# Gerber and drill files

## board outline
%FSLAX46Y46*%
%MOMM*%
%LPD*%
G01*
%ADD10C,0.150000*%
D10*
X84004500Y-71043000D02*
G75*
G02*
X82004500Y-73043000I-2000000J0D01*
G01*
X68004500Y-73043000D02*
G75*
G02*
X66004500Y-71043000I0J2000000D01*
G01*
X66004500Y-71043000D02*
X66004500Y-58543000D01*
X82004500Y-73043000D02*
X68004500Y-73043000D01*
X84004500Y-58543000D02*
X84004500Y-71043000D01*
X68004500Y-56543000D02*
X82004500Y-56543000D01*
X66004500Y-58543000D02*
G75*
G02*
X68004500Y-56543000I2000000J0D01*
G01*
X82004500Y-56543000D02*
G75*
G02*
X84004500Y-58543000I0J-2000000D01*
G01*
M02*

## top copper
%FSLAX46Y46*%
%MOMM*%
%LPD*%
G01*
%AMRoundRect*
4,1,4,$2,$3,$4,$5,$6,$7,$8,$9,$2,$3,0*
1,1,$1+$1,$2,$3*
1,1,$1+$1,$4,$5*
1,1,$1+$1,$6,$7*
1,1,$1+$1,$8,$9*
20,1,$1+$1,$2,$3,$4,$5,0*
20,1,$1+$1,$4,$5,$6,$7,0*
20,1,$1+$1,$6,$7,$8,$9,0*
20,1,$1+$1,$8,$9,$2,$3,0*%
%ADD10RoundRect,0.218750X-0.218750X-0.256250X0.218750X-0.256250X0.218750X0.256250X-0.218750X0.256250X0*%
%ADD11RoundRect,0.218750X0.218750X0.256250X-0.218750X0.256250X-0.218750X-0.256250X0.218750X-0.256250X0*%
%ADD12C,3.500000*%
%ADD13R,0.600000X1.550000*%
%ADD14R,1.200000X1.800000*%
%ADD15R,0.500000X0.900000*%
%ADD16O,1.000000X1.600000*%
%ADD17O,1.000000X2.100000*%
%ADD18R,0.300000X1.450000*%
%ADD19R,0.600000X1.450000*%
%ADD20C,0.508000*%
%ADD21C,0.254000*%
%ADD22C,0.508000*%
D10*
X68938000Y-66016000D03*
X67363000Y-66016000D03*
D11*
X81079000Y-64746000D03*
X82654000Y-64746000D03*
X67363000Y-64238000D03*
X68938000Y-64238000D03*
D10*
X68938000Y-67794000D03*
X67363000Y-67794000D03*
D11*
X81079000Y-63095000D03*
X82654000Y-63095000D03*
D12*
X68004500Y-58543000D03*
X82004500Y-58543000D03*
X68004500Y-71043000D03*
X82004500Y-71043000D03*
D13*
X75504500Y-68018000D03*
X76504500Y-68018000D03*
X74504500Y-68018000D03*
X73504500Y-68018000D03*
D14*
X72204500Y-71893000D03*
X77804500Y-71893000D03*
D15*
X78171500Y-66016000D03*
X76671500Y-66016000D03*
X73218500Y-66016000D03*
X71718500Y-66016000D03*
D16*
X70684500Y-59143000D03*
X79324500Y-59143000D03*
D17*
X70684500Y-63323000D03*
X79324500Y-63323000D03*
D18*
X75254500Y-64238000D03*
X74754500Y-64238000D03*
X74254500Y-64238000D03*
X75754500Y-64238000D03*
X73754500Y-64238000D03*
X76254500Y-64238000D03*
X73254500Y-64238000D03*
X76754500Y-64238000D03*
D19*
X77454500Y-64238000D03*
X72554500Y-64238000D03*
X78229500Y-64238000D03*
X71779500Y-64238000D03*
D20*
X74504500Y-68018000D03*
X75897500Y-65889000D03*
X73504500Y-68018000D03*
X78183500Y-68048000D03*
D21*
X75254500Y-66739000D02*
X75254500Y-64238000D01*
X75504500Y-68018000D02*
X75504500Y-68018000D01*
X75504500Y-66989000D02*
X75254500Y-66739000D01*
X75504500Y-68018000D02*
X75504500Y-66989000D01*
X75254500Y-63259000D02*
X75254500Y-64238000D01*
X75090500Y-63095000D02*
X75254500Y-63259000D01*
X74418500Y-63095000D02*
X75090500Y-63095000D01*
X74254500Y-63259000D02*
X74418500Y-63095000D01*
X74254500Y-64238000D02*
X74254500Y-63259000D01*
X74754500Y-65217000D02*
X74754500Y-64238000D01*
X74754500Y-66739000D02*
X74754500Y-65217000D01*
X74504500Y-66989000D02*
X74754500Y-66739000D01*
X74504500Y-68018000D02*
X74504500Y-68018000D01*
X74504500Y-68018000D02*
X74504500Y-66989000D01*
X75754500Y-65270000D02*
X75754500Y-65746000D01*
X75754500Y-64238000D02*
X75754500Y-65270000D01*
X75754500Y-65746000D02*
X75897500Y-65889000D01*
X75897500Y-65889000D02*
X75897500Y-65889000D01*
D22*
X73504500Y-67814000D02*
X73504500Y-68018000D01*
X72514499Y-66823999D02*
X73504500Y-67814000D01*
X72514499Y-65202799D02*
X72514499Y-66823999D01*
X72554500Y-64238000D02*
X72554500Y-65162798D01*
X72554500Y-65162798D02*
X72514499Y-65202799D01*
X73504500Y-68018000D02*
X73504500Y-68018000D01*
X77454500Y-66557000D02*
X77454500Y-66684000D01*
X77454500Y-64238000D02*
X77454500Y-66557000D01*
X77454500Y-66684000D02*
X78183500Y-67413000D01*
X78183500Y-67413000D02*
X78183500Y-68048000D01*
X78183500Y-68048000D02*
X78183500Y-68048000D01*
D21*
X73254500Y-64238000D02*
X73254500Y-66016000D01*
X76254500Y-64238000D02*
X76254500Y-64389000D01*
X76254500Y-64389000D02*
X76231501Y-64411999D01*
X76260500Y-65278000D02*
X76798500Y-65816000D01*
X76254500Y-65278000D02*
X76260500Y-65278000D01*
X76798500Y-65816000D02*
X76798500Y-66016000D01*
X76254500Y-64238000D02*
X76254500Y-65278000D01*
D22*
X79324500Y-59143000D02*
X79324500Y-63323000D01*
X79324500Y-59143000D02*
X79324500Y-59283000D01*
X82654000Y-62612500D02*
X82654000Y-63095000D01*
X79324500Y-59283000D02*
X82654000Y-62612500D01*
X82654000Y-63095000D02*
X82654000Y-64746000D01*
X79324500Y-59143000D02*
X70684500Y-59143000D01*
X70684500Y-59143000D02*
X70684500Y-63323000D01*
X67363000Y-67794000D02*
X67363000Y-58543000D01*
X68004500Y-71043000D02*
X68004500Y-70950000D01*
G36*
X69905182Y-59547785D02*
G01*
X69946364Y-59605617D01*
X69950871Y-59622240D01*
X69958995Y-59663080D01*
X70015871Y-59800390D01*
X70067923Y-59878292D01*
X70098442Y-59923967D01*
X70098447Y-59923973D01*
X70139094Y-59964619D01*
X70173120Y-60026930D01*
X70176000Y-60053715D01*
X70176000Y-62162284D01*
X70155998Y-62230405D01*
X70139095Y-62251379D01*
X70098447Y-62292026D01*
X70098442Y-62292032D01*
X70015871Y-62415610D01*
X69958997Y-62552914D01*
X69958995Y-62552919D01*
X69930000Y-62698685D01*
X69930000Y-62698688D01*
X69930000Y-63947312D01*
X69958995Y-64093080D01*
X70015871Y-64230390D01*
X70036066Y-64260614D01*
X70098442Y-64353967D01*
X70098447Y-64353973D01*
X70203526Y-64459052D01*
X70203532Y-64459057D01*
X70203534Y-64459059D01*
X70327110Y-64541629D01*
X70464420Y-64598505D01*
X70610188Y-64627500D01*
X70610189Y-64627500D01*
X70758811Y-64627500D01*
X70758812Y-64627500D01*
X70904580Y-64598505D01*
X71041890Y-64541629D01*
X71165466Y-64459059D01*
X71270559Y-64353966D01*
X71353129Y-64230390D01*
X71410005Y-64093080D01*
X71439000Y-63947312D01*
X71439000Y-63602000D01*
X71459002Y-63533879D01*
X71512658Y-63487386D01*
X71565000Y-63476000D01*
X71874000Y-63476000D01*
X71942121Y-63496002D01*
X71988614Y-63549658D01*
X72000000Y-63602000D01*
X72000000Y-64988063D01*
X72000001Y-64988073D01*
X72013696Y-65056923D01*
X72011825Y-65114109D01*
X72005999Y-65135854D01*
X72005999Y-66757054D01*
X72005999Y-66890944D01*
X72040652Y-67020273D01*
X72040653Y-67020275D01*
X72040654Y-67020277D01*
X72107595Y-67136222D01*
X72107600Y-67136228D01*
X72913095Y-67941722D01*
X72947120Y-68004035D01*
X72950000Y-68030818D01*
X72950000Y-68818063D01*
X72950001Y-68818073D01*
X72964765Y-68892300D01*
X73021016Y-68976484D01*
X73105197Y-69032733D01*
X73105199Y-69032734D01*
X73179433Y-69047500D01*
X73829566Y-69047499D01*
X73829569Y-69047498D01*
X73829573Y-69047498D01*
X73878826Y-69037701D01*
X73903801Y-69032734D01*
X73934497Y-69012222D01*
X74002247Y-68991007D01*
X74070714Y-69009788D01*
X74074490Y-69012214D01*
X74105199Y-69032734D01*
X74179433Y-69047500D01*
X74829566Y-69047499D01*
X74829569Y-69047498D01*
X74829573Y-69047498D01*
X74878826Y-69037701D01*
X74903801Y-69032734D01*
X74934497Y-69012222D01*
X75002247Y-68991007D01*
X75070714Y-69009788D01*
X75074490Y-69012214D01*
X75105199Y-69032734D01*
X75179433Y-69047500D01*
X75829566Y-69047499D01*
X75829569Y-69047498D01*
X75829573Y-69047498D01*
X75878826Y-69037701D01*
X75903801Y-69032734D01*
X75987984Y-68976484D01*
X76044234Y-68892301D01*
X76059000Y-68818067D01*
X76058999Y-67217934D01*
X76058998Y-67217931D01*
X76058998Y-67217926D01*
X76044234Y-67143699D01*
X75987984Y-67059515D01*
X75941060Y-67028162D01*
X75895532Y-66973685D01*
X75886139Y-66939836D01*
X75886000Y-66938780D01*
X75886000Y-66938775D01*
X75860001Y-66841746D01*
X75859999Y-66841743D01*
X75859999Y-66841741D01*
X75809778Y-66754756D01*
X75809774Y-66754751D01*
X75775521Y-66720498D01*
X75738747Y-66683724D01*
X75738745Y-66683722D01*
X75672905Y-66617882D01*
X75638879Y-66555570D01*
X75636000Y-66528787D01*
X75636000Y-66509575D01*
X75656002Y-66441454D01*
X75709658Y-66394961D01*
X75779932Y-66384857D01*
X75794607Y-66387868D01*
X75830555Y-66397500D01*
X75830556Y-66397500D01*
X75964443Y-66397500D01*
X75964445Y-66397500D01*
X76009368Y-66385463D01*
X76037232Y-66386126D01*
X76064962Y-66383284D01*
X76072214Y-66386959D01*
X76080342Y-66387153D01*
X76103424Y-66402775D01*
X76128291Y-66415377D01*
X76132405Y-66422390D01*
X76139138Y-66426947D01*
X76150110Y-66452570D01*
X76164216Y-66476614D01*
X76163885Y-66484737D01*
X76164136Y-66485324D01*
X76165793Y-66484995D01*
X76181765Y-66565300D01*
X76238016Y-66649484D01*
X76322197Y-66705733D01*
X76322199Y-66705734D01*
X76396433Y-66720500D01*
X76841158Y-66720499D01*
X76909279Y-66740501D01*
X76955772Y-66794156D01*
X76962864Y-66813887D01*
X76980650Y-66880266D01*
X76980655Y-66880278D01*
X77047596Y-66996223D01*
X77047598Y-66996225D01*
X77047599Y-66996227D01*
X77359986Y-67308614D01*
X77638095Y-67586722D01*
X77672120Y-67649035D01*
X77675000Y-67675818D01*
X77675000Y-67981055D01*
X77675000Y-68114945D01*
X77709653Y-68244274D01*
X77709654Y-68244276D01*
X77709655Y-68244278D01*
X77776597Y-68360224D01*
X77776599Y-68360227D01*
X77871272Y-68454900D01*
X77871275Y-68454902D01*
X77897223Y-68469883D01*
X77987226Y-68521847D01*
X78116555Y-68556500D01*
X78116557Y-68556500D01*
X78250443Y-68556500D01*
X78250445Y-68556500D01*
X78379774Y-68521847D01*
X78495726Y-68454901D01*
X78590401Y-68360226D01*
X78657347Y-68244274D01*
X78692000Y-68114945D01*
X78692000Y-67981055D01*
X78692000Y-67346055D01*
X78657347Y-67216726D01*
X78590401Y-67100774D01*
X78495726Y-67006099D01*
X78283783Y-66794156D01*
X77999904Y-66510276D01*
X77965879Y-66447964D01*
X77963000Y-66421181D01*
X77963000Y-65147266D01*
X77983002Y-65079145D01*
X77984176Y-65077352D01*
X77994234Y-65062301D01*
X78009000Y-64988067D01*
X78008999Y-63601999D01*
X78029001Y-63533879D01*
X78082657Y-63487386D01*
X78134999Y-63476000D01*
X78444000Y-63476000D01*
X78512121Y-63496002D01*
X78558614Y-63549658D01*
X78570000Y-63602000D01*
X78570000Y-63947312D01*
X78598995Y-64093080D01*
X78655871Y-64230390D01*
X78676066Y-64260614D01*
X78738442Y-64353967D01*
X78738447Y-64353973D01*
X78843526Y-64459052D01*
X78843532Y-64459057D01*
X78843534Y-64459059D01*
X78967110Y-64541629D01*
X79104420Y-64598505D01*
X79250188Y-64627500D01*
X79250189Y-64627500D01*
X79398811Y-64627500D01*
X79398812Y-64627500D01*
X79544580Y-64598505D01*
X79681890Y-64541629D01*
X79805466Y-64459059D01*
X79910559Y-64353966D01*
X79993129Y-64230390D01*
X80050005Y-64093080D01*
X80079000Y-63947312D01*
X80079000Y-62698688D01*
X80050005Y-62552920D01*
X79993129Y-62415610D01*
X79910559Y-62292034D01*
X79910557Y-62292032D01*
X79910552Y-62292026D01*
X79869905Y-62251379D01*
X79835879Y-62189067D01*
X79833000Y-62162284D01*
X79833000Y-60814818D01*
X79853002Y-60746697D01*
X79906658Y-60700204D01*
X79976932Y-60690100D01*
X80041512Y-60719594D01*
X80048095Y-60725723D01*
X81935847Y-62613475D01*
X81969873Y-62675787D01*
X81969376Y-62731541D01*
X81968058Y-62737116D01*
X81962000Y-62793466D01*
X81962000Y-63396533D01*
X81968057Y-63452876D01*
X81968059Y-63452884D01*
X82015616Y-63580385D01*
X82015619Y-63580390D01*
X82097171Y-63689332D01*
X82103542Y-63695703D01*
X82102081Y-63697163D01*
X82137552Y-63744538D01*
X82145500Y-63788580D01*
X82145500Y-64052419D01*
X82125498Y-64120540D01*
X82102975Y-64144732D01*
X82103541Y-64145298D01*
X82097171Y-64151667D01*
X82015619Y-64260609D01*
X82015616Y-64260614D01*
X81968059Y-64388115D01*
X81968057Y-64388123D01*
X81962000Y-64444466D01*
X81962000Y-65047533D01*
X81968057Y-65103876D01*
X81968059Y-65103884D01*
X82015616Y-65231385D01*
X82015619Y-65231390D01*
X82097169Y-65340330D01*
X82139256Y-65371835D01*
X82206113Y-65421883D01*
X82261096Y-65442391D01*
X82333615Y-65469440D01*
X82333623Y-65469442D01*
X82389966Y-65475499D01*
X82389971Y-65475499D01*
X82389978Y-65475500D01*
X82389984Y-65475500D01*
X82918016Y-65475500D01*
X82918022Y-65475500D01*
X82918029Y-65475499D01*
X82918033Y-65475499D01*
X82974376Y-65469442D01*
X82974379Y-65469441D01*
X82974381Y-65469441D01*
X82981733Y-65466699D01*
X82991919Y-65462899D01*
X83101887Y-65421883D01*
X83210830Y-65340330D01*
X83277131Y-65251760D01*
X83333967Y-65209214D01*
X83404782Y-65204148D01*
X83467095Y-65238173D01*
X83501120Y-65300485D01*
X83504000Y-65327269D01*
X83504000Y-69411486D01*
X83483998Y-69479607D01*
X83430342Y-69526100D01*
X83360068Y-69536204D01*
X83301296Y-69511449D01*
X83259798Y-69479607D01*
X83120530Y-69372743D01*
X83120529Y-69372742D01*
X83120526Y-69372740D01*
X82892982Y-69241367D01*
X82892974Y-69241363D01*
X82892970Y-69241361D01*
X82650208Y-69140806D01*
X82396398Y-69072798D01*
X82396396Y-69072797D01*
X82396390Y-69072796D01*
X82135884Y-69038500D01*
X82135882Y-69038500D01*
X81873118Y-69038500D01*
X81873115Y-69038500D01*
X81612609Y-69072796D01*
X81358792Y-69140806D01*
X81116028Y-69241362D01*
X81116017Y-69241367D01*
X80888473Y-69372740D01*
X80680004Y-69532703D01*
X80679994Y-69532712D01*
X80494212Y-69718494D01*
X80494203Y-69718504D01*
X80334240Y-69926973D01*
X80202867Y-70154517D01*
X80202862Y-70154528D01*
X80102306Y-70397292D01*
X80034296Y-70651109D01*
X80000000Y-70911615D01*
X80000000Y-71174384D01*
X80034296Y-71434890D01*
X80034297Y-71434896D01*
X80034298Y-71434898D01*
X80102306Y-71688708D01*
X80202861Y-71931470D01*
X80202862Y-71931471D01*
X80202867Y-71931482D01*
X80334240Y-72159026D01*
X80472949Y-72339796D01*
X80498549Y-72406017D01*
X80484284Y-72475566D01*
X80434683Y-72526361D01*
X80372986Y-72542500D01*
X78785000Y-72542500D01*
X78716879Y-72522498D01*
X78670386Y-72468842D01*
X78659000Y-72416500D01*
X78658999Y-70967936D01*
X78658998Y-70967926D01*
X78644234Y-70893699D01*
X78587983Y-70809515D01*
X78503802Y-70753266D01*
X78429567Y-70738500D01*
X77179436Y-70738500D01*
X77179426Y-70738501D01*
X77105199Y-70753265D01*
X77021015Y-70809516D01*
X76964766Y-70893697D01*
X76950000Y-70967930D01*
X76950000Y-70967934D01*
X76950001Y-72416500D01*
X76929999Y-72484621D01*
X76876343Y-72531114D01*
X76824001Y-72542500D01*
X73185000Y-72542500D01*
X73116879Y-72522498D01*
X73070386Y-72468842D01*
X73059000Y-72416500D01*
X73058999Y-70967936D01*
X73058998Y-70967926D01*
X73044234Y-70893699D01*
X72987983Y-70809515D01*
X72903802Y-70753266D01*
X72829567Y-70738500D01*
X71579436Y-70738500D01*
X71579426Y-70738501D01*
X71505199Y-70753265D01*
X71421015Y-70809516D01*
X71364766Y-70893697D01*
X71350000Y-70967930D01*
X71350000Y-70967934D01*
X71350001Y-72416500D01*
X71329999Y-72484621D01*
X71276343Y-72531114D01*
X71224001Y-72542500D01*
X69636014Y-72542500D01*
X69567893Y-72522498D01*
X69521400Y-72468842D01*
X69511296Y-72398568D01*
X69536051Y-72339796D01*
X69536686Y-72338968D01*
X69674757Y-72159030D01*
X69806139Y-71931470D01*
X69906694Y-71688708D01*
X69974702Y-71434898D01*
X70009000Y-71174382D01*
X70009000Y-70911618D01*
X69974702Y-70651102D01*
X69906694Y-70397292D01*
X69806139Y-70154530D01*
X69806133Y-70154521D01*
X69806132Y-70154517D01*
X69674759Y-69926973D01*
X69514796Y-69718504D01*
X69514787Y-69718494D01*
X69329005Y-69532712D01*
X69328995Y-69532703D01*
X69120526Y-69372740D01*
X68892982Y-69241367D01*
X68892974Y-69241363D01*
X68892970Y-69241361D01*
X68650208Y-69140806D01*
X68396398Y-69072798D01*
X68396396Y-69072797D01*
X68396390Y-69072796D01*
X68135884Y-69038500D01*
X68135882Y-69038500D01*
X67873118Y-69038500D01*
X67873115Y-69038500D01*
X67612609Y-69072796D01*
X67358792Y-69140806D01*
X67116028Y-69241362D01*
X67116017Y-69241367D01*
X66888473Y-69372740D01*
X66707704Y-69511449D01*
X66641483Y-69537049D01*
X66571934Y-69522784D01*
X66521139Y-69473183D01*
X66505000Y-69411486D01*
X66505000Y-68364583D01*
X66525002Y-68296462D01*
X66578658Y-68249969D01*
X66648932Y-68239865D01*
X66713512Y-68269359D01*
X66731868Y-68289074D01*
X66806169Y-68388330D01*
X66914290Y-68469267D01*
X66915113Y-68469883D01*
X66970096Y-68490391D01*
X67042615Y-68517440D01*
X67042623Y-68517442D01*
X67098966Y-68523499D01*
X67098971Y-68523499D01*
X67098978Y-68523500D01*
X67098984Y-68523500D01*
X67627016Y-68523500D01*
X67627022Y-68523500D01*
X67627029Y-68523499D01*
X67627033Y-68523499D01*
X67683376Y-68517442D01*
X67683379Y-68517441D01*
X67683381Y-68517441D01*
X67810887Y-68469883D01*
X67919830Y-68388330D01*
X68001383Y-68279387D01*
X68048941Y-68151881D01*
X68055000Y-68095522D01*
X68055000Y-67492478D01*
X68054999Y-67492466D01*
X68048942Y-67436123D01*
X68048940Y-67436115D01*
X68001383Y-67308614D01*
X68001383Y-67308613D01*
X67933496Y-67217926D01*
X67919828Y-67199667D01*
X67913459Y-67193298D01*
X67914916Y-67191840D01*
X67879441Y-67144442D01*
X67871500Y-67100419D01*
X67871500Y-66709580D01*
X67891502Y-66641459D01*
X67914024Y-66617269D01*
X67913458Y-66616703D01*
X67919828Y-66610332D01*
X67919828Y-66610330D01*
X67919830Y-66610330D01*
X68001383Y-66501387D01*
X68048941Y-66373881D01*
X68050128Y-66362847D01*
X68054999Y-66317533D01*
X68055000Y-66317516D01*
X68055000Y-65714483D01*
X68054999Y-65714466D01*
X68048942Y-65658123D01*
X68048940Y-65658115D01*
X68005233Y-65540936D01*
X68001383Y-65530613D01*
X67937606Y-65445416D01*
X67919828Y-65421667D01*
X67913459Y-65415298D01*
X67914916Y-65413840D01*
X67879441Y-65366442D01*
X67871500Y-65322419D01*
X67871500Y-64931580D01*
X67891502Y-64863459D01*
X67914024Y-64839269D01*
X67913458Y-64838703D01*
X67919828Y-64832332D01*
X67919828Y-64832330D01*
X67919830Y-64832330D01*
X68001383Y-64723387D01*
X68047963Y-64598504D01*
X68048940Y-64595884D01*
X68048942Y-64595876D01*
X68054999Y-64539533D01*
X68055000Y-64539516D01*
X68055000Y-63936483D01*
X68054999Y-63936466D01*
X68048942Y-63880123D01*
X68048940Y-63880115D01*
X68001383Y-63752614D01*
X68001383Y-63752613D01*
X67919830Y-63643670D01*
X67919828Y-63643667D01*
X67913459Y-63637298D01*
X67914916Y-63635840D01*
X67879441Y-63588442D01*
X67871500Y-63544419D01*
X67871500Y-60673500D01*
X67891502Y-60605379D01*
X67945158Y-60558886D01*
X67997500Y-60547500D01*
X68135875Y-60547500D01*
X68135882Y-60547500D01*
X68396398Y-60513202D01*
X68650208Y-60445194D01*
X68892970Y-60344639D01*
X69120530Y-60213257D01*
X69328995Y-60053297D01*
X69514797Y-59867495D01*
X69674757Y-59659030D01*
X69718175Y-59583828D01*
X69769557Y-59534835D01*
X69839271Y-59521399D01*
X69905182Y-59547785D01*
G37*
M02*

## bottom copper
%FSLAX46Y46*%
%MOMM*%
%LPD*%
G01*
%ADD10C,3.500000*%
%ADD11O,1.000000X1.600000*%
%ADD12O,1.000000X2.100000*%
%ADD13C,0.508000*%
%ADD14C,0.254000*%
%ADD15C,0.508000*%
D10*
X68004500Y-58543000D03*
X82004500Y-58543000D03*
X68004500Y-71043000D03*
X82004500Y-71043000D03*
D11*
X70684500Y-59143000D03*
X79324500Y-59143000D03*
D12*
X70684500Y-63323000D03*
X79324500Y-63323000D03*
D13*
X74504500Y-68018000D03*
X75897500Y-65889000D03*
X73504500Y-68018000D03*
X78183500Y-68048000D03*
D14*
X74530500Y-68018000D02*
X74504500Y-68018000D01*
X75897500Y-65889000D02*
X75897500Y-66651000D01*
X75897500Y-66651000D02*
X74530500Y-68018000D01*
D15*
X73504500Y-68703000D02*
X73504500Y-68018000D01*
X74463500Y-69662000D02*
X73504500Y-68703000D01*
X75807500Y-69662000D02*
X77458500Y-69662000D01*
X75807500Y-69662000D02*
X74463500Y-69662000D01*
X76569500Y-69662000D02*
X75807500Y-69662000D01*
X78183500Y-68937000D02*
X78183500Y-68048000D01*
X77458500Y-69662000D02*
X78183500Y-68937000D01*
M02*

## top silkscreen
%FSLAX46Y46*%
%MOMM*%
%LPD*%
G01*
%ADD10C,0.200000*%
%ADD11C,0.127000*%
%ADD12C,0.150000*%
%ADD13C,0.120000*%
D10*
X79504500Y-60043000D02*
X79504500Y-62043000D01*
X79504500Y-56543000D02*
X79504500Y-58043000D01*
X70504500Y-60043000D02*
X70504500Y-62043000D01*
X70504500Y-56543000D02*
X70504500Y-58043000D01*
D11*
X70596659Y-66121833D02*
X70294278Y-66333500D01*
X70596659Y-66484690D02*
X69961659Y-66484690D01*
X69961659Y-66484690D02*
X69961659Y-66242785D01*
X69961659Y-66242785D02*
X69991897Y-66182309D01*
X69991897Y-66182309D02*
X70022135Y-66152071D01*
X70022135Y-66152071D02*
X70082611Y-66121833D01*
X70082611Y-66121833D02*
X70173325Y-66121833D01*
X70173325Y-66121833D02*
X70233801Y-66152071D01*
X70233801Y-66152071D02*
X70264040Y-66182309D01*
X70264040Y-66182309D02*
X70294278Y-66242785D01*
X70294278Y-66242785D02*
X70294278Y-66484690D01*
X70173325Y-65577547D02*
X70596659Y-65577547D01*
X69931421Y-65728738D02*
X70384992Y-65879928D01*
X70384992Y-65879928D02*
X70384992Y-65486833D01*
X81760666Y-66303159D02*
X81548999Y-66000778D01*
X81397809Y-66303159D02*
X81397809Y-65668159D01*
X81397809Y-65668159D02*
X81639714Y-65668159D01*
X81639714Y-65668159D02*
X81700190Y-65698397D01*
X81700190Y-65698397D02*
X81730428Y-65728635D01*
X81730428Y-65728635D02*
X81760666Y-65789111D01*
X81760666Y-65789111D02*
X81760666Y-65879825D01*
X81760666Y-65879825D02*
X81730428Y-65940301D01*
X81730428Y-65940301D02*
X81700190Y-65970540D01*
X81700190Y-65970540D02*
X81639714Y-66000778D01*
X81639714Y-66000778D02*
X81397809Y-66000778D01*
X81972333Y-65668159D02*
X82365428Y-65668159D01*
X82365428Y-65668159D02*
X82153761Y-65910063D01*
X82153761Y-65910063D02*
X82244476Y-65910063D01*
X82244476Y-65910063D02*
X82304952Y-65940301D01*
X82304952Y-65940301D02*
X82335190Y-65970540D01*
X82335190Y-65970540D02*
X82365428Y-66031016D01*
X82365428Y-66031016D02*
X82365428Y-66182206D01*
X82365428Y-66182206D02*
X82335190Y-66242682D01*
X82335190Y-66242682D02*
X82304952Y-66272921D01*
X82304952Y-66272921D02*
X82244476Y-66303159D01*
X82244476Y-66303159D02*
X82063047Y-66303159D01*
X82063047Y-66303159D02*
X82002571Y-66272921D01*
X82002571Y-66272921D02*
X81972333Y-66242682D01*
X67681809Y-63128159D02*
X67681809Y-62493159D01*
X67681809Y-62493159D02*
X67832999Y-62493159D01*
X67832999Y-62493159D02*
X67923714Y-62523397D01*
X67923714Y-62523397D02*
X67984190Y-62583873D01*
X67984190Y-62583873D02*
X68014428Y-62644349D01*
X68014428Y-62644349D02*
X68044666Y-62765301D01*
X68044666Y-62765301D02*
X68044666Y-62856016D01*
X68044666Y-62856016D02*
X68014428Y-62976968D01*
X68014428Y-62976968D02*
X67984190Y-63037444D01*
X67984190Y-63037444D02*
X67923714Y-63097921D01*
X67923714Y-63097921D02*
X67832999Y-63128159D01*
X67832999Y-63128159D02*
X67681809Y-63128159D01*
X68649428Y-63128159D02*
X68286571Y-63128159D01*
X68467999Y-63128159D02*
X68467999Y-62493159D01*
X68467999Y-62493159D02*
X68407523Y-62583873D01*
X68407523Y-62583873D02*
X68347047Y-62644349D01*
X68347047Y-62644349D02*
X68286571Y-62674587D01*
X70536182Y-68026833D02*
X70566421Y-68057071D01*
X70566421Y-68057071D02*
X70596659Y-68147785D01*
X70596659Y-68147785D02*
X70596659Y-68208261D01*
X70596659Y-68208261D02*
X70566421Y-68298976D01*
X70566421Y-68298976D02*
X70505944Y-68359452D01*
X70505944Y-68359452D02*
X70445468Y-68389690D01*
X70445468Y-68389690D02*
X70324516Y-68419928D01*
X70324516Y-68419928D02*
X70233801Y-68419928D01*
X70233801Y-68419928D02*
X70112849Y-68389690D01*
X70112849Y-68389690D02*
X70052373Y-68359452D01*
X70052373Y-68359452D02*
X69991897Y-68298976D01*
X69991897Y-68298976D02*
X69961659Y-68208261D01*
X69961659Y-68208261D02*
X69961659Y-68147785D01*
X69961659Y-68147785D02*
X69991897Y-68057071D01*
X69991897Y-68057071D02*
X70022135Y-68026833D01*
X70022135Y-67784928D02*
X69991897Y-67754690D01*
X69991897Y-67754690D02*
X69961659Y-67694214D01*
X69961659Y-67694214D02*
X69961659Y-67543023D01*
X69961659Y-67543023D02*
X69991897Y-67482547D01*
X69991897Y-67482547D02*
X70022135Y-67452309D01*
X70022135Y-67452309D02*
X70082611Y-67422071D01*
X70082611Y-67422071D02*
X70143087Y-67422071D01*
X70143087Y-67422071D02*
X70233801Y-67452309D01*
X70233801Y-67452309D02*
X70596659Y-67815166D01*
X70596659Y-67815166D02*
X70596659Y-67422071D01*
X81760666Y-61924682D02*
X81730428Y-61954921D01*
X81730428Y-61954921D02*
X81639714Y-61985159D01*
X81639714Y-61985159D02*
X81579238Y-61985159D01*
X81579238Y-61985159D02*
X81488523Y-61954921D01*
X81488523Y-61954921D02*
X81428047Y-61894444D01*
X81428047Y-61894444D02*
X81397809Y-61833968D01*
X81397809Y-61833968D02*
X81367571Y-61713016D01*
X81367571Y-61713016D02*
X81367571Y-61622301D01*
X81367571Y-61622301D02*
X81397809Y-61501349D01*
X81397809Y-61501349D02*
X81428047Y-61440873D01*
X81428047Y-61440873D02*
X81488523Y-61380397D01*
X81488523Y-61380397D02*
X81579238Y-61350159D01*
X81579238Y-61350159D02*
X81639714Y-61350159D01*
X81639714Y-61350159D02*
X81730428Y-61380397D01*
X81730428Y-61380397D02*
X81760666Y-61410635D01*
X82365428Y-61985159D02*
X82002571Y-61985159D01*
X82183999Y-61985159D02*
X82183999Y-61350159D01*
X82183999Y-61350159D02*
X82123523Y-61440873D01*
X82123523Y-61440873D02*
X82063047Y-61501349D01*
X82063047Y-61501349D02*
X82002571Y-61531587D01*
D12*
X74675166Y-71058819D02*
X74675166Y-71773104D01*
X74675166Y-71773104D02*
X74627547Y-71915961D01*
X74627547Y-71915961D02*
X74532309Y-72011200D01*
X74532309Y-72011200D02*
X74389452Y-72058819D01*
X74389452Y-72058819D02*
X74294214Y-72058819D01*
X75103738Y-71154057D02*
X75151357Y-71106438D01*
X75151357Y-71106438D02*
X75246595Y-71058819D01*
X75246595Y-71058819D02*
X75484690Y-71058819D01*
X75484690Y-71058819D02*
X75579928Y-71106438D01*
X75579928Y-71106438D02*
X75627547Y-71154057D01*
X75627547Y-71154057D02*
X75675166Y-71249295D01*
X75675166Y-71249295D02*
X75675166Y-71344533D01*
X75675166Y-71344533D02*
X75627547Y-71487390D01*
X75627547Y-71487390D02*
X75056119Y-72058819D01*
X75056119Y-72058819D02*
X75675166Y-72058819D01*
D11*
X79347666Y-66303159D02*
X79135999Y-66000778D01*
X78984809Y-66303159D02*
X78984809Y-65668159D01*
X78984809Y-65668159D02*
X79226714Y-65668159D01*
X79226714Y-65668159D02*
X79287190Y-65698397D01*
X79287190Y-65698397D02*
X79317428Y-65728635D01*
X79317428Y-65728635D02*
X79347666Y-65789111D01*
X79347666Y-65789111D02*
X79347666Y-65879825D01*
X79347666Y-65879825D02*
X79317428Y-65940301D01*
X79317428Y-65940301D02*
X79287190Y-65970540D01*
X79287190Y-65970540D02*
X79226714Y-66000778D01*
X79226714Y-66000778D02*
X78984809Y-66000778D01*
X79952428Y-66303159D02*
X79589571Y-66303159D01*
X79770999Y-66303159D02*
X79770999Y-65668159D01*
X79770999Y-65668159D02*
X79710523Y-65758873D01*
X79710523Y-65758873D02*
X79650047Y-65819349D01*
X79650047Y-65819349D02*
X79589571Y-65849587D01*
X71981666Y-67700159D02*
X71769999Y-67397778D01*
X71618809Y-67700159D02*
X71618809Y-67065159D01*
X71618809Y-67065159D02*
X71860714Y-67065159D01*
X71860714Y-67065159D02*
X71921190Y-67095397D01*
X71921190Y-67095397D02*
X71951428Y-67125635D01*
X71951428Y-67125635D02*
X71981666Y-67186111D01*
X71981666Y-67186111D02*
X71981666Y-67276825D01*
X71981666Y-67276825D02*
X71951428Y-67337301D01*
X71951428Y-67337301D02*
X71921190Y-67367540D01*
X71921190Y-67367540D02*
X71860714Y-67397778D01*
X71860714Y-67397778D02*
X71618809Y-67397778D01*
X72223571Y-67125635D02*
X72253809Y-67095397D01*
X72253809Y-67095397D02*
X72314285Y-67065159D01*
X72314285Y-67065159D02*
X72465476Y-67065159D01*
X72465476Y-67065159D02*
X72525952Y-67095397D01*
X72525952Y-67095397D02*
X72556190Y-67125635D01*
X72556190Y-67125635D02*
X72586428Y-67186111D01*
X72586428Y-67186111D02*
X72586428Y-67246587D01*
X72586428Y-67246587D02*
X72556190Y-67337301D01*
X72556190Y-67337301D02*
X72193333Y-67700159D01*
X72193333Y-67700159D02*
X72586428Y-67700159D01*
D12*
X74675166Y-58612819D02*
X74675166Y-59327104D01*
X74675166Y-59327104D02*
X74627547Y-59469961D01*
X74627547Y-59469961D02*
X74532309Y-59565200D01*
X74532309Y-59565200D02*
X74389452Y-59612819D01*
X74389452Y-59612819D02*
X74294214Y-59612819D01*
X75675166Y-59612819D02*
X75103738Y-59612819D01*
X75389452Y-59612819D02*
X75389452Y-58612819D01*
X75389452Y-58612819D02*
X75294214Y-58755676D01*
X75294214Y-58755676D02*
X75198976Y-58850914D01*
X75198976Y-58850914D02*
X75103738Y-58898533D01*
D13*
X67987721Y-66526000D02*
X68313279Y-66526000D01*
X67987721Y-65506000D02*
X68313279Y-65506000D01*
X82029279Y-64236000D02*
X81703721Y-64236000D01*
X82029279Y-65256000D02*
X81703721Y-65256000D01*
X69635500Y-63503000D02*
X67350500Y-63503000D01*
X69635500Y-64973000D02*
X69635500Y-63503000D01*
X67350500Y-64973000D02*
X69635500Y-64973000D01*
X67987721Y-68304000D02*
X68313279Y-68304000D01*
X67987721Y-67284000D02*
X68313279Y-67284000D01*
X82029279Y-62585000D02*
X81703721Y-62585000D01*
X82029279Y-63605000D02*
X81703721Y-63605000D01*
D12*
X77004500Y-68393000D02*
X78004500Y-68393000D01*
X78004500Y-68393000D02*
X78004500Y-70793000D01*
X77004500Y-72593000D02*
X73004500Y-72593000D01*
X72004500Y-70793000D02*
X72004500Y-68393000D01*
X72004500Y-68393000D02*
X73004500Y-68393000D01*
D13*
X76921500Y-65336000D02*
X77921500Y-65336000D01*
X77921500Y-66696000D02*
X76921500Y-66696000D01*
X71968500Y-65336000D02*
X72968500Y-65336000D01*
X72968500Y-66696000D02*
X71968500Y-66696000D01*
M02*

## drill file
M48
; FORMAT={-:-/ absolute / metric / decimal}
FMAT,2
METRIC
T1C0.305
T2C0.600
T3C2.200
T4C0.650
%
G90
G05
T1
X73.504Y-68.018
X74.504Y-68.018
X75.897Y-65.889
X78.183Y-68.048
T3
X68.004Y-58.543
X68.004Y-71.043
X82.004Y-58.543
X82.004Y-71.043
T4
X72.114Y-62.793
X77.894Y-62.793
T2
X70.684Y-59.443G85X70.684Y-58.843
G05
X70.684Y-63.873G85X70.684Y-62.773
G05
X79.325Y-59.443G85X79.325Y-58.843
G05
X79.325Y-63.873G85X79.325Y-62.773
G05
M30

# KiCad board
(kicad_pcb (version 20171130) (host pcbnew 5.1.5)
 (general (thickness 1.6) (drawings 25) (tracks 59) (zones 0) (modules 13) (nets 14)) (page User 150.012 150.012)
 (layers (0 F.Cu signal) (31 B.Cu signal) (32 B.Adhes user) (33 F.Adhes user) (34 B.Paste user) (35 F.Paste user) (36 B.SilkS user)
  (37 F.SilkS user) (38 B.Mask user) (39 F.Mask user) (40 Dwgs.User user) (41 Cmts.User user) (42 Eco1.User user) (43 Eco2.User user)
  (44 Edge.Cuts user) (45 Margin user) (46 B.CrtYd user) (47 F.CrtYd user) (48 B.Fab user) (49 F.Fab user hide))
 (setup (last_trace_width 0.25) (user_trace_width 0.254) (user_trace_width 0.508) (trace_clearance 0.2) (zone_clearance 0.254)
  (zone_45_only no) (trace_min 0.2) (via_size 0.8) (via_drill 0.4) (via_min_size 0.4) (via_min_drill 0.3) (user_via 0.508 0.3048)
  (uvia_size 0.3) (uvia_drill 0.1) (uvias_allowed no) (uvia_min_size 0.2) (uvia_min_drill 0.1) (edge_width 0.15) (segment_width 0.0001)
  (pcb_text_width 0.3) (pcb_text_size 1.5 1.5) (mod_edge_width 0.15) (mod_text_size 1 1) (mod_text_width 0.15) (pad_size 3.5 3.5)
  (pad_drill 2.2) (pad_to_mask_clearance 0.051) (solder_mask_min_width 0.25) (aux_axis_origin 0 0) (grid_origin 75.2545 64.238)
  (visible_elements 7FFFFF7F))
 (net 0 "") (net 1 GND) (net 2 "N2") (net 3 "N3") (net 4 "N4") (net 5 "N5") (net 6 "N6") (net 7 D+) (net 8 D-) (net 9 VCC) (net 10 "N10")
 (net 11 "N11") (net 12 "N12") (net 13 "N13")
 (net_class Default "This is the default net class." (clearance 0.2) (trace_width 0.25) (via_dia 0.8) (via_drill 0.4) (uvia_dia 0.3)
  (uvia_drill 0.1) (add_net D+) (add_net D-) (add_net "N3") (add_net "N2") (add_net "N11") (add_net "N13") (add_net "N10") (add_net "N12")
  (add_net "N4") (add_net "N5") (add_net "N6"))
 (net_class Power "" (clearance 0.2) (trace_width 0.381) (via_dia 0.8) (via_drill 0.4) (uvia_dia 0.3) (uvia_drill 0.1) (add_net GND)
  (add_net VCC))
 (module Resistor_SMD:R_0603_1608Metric (layer F.Cu) (at 68.1505 66.016)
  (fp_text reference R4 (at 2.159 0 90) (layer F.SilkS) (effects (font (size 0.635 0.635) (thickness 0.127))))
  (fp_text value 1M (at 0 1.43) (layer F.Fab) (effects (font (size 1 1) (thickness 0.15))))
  (fp_line (start -0.162779 0.51) (end 0.162779 0.51) (layer F.SilkS) (width 0.12))
  (fp_line (start -0.162779 -0.51) (end 0.162779 -0.51) (layer F.SilkS) (width 0.12))
  (pad 2 smd roundrect (at 0.7875 0) (size 0.875 0.95) (layers F.Cu F.Paste F.Mask) (roundrect_rratio 0.25) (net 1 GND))
  (pad 1 smd roundrect (at -0.7875 0) (size 0.875 0.95) (layers F.Cu F.Paste F.Mask) (roundrect_rratio 0.25) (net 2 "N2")))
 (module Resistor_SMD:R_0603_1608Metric (layer F.Cu) (at 81.8665 64.746 180)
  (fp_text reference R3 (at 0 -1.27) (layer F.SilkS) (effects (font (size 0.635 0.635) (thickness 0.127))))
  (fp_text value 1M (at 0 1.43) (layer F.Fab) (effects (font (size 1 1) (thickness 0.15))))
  (fp_line (start -0.162779 0.51) (end 0.162779 0.51) (layer F.SilkS) (width 0.12))
  (fp_line (start -0.162779 -0.51) (end 0.162779 -0.51) (layer F.SilkS) (width 0.12))
  (pad 2 smd roundrect (at 0.7875 0 180) (size 0.875 0.95) (layers F.Cu F.Paste F.Mask) (roundrect_rratio 0.25) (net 1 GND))
  (pad 1 smd roundrect (at -0.7875 0 180) (size 0.875 0.95) (layers F.Cu F.Paste F.Mask) (roundrect_rratio 0.25) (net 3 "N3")))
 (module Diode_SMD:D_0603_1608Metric (layer F.Cu) (at 68.1505 64.238 180)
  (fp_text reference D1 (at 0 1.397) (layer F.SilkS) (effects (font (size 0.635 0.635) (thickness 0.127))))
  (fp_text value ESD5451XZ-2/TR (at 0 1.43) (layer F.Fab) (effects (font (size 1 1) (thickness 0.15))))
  (fp_line (start -1.485 0.735) (end 0.8 0.735) (layer F.SilkS) (width 0.12))
  (fp_line (start -1.485 -0.735) (end -1.485 0.735) (layer F.SilkS) (width 0.12))
  (fp_line (start 0.8 -0.735) (end -1.485 -0.735) (layer F.SilkS) (width 0.12))
  (pad 2 smd roundrect (at 0.7875 0 180) (size 0.875 0.95) (layers F.Cu F.Paste F.Mask) (roundrect_rratio 0.25) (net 2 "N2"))
  (pad 1 smd roundrect (at -0.7875 0 180) (size 0.875 0.95) (layers F.Cu F.Paste F.Mask) (roundrect_rratio 0.25) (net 1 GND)))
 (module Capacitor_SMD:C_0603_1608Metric (layer F.Cu) (at 68.1505 67.794)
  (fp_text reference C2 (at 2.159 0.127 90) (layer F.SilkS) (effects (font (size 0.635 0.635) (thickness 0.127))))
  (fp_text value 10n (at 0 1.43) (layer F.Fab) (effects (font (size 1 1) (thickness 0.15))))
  (fp_line (start -0.162779 0.51) (end 0.162779 0.51) (layer F.SilkS) (width 0.12))
  (fp_line (start -0.162779 -0.51) (end 0.162779 -0.51) (layer F.SilkS) (width 0.12))
  (pad 2 smd roundrect (at 0.7875 0) (size 0.875 0.95) (layers F.Cu F.Paste F.Mask) (roundrect_rratio 0.25) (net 1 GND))
  (pad 1 smd roundrect (at -0.7875 0) (size 0.875 0.95) (layers F.Cu F.Paste F.Mask) (roundrect_rratio 0.25) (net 2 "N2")))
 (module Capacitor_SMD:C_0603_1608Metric (layer F.Cu) (at 81.8665 63.095 180)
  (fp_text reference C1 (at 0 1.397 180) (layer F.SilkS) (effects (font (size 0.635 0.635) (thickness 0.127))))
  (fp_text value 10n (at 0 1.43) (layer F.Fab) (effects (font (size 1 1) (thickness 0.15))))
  (fp_line (start -0.162779 0.51) (end 0.162779 0.51) (layer F.SilkS) (width 0.12))
  (fp_line (start -0.162779 -0.51) (end 0.162779 -0.51) (layer F.SilkS) (width 0.12))
  (pad 2 smd roundrect (at 0.7875 0 180) (size 0.875 0.95) (layers F.Cu F.Paste F.Mask) (roundrect_rratio 0.25) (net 1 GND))
  (pad 1 smd roundrect (at -0.7875 0 180) (size 0.875 0.95) (layers F.Cu F.Paste F.Mask) (roundrect_rratio 0.25) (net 3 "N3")))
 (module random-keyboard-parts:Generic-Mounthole (layer F.Cu) (at 68.0045 58.543)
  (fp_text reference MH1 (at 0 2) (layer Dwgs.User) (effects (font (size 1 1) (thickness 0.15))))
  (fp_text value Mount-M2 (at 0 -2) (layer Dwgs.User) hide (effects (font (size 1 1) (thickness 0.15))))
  (pad 1 thru_hole circle (at 0 0) (size 3.5 3.5) (drill 2.2) (layers *.Cu *.Mask) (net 2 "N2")))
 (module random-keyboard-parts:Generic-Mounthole (layer F.Cu) (at 82.0045 58.543)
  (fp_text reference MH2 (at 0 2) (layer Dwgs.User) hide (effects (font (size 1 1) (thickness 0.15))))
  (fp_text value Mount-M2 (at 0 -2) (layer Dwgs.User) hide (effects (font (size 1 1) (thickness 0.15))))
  (pad 1 thru_hole circle (at 0 0) (size 3.5 3.5) (drill 2.2) (layers *.Cu F.Mask) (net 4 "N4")))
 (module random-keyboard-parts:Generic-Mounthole (layer F.Cu) (at 68.0045 71.043)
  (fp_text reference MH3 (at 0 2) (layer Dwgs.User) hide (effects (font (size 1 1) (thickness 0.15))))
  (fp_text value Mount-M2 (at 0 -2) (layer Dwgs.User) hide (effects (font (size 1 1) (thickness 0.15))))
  (pad 1 thru_hole circle (at 0 0) (size 3.5 3.5) (drill 2.2) (layers *.Cu F.Mask) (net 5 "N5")))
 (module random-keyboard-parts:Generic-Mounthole (layer F.Cu) (at 82.0045 71.043)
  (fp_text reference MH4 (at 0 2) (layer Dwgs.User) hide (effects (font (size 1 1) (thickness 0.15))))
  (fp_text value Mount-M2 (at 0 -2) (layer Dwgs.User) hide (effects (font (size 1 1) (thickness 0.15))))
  (pad 1 thru_hole circle (at 0 0) (size 3.5 3.5) (drill 2.2) (layers *.Cu F.Mask) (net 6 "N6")))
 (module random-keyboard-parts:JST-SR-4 (layer F.Cu) (at 75.0045 72.793)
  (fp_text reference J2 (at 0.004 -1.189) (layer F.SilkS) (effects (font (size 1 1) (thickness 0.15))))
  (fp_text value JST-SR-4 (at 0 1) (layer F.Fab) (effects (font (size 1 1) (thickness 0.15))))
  (fp_line (start 2 -4.4) (end 3 -4.4) (layer F.SilkS) (width 0.15))
  (fp_line (start 3 -4.4) (end 3 -2) (layer F.SilkS) (width 0.15))
  (fp_line (start 2 -0.2) (end -2 -0.2) (layer F.SilkS) (width 0.15))
  (fp_line (start -3 -2) (end -3 -4.4) (layer F.SilkS) (width 0.15))
  (fp_line (start -3 -4.4) (end -2 -4.4) (layer F.SilkS) (width 0.15))
  (pad 3 smd rect (at 0.5 -4.775) (size 0.6 1.55) (layers F.Cu F.Paste F.Mask) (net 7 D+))
  (pad 4 smd rect (at 1.5 -4.775) (size 0.6 1.55) (layers F.Cu F.Paste F.Mask) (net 1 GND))
  (pad 2 smd rect (at -0.5 -4.775) (size 0.6 1.55) (layers F.Cu F.Paste F.Mask) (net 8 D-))
  (pad 1 smd rect (at -1.5 -4.775) (size 0.6 1.55) (layers F.Cu F.Paste F.Mask) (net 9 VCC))
  (pad "" smd rect (at -2.8 -0.9) (size 1.2 1.8) (layers F.Cu F.Paste F.Mask))
  (pad "" smd rect (at 2.8 -0.9) (size 1.2 1.8) (layers F.Cu F.Paste F.Mask)))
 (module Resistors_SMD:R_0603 (layer F.Cu) (at 77.4215 66.016)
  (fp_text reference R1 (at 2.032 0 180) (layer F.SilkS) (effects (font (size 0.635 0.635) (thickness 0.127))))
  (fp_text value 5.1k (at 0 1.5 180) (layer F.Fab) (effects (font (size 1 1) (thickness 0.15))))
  (fp_line (start -0.5 -0.68) (end 0.5 -0.68) (layer F.SilkS) (width 0.12))
  (fp_line (start 0.5 0.68) (end -0.5 0.68) (layer F.SilkS) (width 0.12))
  (pad 2 smd rect (at 0.75 0) (size 0.5 0.9) (layers F.Cu F.Paste F.Mask) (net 1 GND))
  (pad 1 smd rect (at -0.75 0) (size 0.5 0.9) (layers F.Cu F.Paste F.Mask) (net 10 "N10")))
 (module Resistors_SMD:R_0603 (layer F.Cu) (at 72.4685 66.016 180)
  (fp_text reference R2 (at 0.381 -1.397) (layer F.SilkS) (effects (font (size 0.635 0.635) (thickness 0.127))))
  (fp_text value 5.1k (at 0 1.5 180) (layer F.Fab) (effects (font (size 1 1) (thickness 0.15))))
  (fp_line (start 0.5 0.68) (end -0.5 0.68) (layer F.SilkS) (width 0.12))
  (fp_line (start -0.5 -0.68) (end 0.5 -0.68) (layer F.SilkS) (width 0.12))
  (pad 1 smd rect (at -0.75 0 180) (size 0.5 0.9) (layers F.Cu F.Paste F.Mask) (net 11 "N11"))
  (pad 2 smd rect (at 0.75 0 180) (size 0.5 0.9) (layers F.Cu F.Paste F.Mask) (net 1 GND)))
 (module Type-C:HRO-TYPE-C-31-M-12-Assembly (layer F.Cu) (at 75.0045 56.543 180)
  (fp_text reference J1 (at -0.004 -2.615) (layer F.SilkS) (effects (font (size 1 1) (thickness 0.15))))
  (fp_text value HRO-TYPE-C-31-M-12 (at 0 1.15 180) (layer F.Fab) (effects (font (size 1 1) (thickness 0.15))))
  (pad 13 thru_hole oval (at 4.32 -2.6 180) (size 1 1.6) (drill oval 0.6 1.2) (layers *.Cu F.Mask) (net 3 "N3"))
  (pad 13 thru_hole oval (at -4.32 -2.6 180) (size 1 1.6) (drill oval 0.6 1.2) (layers *.Cu F.Mask) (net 3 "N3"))
  (pad 13 thru_hole oval (at 4.32 -6.78 180) (size 1 2.1) (drill oval 0.6 1.7) (layers *.Cu F.Mask) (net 3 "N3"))
  (pad 13 thru_hole oval (at -4.32 -6.78 180) (size 1 2.1) (drill oval 0.6 1.7) (layers *.Cu F.Mask) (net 3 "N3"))
  (pad "" np_thru_hole circle (at -2.89 -6.25 180) (size 0.65 0.65) (drill 0.65) (layers *.Cu *.Mask))
  (pad "" np_thru_hole circle (at 2.89 -6.25 180) (size 0.65 0.65) (drill 0.65) (layers *.Cu *.Mask))
  (pad 6 smd rect (at -0.25 -7.695 180) (size 0.3 1.45) (layers F.Cu F.Paste F.Mask) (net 7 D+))
  (pad 7 smd rect (at 0.25 -7.695 180) (size 0.3 1.45) (layers F.Cu F.Paste F.Mask) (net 8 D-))
  (pad 8 smd rect (at 0.75 -7.695 180) (size 0.3 1.45) (layers F.Cu F.Paste F.Mask) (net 7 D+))
  (pad 5 smd rect (at -0.75 -7.695 180) (size 0.3 1.45) (layers F.Cu F.Paste F.Mask) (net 8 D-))
  (pad 9 smd rect (at 1.25 -7.695 180) (size 0.3 1.45) (layers F.Cu F.Paste F.Mask) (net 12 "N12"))
  (pad 4 smd rect (at -1.25 -7.695 180) (size 0.3 1.45) (layers F.Cu F.Paste F.Mask) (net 10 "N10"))
  (pad 10 smd rect (at 1.75 -7.695 180) (size 0.3 1.45) (layers F.Cu F.Paste F.Mask) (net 11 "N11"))
  (pad 3 smd rect (at -1.75 -7.695 180) (size 0.3 1.45) (layers F.Cu F.Paste F.Mask) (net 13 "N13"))
  (pad 2 smd rect (at -2.45 -7.695 180) (size 0.6 1.45) (layers F.Cu F.Paste F.Mask) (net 9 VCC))
  (pad 11 smd rect (at 2.45 -7.695 180) (size 0.6 1.45) (layers F.Cu F.Paste F.Mask) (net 9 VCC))
  (pad 1 smd rect (at -3.225 -7.695 180) (size 0.6 1.45) (layers F.Cu F.Paste F.Mask) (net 1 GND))
  (pad 12 smd rect (at 3.225 -7.695 180) (size 0.6 1.45) (layers F.Cu F.Paste F.Mask) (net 1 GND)))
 (gr_line (start 79.5045 60.043) (end 79.5045 62.043) (layer F.SilkS) (width 0.2))
 (gr_line (start 79.5045 56.543) (end 79.5045 58.043) (layer F.SilkS) (width 0.2))
 (gr_line (start 70.5045 60.043) (end 70.5045 62.043) (layer F.SilkS) (width 0.2))
 (gr_line (start 70.5045 56.543) (end 70.5045 58.043) (layer F.SilkS) (width 0.2))
 (gr_arc (start 82.0045 71.043) (end 82.0045 73.043) (angle -90) (layer Edge.Cuts) (width 0.15))
 (gr_arc (start 68.0045 71.043) (end 66.0045 71.043) (angle -90) (layer Edge.Cuts) (width 0.15))
 (gr_line (start 66.0045 71.043) (end 66.0045 58.543) (layer Edge.Cuts) (width 0.15))
 (gr_line (start 82.0045 73.043) (end 68.0045 73.043) (layer Edge.Cuts) (width 0.15))
 (gr_line (start 84.0045 58.543) (end 84.0045 71.043) (layer Edge.Cuts) (width 0.15))
 (gr_line (start 68.0045 56.543) (end 82.0045 56.543) (layer Edge.Cuts) (width 0.15))
 (gr_arc (start 68.0045 58.543) (end 68.0045 56.543) (angle -90) (layer Edge.Cuts) (width 0.15))
 (gr_arc (start 82.0045 58.543) (end 84.0045 58.543) (angle -90) (layer Edge.Cuts) (width 0.15))
 (segment (start 75.2545 66.739) (end 75.2545 64.238) (width 0.254) (layer F.Cu) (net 7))
 (segment (start 75.5045 68.018) (end 75.5045 68.018) (width 0.254) (layer F.Cu) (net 7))
 (segment (start 75.5045 66.989) (end 75.2545 66.739) (width 0.254) (layer F.Cu) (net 7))
 (segment (start 75.5045 68.018) (end 75.5045 66.989) (width 0.254) (layer F.Cu) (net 7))
 (segment (start 75.2545 63.259) (end 75.2545 64.238) (width 0.254) (layer F.Cu) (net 7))
 (segment (start 75.0905 63.095) (end 75.2545 63.259) (width 0.254) (layer F.Cu) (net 7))
 (segment (start 74.4185 63.095) (end 75.0905 63.095) (width 0.254) (layer F.Cu) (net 7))
 (segment (start 74.2545 63.259) (end 74.4185 63.095) (width 0.254) (layer F.Cu) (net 7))
 (segment (start 74.2545 64.238) (end 74.2545 63.259) (width 0.254) (layer F.Cu) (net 7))
 (segment (start 74.7545 65.217) (end 74.7545 64.238) (width 0.254) (layer F.Cu) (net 8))
 (segment (start 74.7545 66.739) (end 74.7545 65.217) (width 0.254) (layer F.Cu) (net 8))
 (segment (start 74.5045 66.989) (end 74.7545 66.739) (width 0.254) (layer F.Cu) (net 8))
 (segment (start 74.5045 68.018) (end 74.5045 68.018) (width 0.254) (layer F.Cu) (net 8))
 (segment (start 74.5045 68.018) (end 74.5045 66.989) (width 0.254) (layer F.Cu) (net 8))
 (via (at 74.5045 68.018) (size 0.508) (drill 0.3048) (layers F.Cu B.Cu) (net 8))
 (segment (start 75.7545 65.27) (end 75.7545 65.746) (width 0.254) (layer F.Cu) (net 8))
 (segment (start 75.7545 64.238) (end 75.7545 65.27) (width 0.254) (layer F.Cu) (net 8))
 (segment (start 75.7545 65.746) (end 75.8975 65.889) (width 0.254) (layer F.Cu) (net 8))
 (segment (start 75.8975 65.889) (end 75.8975 65.889) (width 0.254) (layer F.Cu) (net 8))
 (via (at 75.8975 65.889) (size 0.508) (drill 0.3048) (layers F.Cu B.Cu) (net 8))
 (segment (start 74.5305 68.018) (end 74.5045 68.018) (width 0.254) (layer B.Cu) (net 8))
 (segment (start 75.8975 65.889) (end 75.8975 66.651) (width 0.254) (layer B.Cu) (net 8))
 (segment (start 75.8975 66.651) (end 74.5305 68.018) (width 0.254) (layer B.Cu) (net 8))
 (segment (start 73.5045 67.814) (end 73.5045 68.018) (width 0.508) (layer F.Cu) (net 9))
 (segment (start 72.514499 66.823999) (end 73.5045 67.814) (width 0.508) (layer F.Cu) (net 9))
 (segment (start 72.514499 65.202799) (end 72.514499 66.823999) (width 0.508) (layer F.Cu) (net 9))
 (segment (start 72.5545 64.238) (end 72.5545 65.162798) (width 0.508) (layer F.Cu) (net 9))
 (segment (start 72.5545 65.162798) (end 72.514499 65.202799) (width 0.508) (layer F.Cu) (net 9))
 (segment (start 73.5045 68.018) (end 73.5045 68.018) (width 0.508) (layer F.Cu) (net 9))
 (via (at 73.5045 68.018) (size 0.508) (drill 0.3048) (layers F.Cu B.Cu) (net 9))
 (segment (start 73.5045 68.703) (end 73.5045 68.018) (width 0.508) (layer B.Cu) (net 9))
 (segment (start 74.4635 69.662) (end 73.5045 68.703) (width 0.508) (layer B.Cu) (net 9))
 (segment (start 77.4545 66.557) (end 77.4545 66.684) (width 0.508) (layer F.Cu) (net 9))
 (segment (start 77.4545 64.238) (end 77.4545 66.557) (width 0.508) (layer F.Cu) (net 9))
 (segment (start 77.4545 66.684) (end 78.1835 67.413) (width 0.508) (layer F.Cu) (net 9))
 (segment (start 78.1835 67.413) (end 78.1835 68.048) (width 0.508) (layer F.Cu) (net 9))
 (segment (start 78.1835 68.048) (end 78.1835 68.048) (width 0.508) (layer F.Cu) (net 9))
 (via (at 78.1835 68.048) (size 0.508) (drill 0.3048) (layers F.Cu B.Cu) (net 9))
 (segment (start 75.8075 69.662) (end 77.4585 69.662) (width 0.508) (layer B.Cu) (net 9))
 (segment (start 75.8075 69.662) (end 74.4635 69.662) (width 0.508) (layer B.Cu) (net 9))
 (segment (start 76.5695 69.662) (end 75.8075 69.662) (width 0.508) (layer B.Cu) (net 9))
 (segment (start 78.1835 68.937) (end 78.1835 68.048) (width 0.508) (layer B.Cu) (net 9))
 (segment (start 77.4585 69.662) (end 78.1835 68.937) (width 0.508) (layer B.Cu) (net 9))
 (segment (start 73.2545 64.238) (end 73.2545 66.016) (width 0.254) (layer F.Cu) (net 11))
 (segment (start 76.2545 64.238) (end 76.2545 64.389) (width 0.254) (layer F.Cu) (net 10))
 (segment (start 76.2545 64.389) (end 76.231501 64.411999) (width 0.254) (layer F.Cu) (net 10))
 (segment (start 76.2605 65.278) (end 76.7985 65.816) (width 0.254) (layer F.Cu) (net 10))
 (segment (start 76.2545 65.278) (end 76.2605 65.278) (width 0.254) (layer F.Cu) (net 10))
 (segment (start 76.7985 65.816) (end 76.7985 66.016) (width 0.254) (layer F.Cu) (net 10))
 (segment (start 76.2545 64.238) (end 76.2545 65.278) (width 0.254) (layer F.Cu) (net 10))
 (segment (start 79.3245 59.143) (end 79.3245 63.323) (width 0.508) (layer F.Cu) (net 3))
 (segment (start 79.3245 59.143) (end 79.3245 59.283) (width 0.508) (layer F.Cu) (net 3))
 (segment (start 82.654 62.6125) (end 82.654 63.095) (width 0.508) (layer F.Cu) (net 3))
 (segment (start 79.3245 59.283) (end 82.654 62.6125) (width 0.508) (layer F.Cu) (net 3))
 (segment (start 82.654 63.095) (end 82.654 64.746) (width 0.508) (layer F.Cu) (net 3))
 (segment (start 79.3245 59.143) (end 70.6845 59.143) (width 0.508) (layer F.Cu) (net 3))
 (segment (start 70.6845 59.143) (end 70.6845 63.323) (width 0.508) (layer F.Cu) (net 3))
 (segment (start 67.363 67.794) (end 67.363 58.543) (width 0.508) (layer F.Cu) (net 2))
 (segment (start 68.0045 71.043) (end 68.0045 70.95) (width 0.508) (layer F.Cu) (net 5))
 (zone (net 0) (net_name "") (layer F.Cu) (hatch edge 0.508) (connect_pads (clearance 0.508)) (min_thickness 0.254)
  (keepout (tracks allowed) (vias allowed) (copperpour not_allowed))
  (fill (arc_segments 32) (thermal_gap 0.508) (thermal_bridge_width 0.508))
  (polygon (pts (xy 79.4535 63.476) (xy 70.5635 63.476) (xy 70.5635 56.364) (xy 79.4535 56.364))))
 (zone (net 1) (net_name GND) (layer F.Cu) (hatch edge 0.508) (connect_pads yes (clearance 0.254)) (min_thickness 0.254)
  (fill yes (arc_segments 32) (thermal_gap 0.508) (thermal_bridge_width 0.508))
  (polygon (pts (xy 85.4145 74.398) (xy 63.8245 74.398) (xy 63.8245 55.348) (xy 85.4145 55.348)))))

